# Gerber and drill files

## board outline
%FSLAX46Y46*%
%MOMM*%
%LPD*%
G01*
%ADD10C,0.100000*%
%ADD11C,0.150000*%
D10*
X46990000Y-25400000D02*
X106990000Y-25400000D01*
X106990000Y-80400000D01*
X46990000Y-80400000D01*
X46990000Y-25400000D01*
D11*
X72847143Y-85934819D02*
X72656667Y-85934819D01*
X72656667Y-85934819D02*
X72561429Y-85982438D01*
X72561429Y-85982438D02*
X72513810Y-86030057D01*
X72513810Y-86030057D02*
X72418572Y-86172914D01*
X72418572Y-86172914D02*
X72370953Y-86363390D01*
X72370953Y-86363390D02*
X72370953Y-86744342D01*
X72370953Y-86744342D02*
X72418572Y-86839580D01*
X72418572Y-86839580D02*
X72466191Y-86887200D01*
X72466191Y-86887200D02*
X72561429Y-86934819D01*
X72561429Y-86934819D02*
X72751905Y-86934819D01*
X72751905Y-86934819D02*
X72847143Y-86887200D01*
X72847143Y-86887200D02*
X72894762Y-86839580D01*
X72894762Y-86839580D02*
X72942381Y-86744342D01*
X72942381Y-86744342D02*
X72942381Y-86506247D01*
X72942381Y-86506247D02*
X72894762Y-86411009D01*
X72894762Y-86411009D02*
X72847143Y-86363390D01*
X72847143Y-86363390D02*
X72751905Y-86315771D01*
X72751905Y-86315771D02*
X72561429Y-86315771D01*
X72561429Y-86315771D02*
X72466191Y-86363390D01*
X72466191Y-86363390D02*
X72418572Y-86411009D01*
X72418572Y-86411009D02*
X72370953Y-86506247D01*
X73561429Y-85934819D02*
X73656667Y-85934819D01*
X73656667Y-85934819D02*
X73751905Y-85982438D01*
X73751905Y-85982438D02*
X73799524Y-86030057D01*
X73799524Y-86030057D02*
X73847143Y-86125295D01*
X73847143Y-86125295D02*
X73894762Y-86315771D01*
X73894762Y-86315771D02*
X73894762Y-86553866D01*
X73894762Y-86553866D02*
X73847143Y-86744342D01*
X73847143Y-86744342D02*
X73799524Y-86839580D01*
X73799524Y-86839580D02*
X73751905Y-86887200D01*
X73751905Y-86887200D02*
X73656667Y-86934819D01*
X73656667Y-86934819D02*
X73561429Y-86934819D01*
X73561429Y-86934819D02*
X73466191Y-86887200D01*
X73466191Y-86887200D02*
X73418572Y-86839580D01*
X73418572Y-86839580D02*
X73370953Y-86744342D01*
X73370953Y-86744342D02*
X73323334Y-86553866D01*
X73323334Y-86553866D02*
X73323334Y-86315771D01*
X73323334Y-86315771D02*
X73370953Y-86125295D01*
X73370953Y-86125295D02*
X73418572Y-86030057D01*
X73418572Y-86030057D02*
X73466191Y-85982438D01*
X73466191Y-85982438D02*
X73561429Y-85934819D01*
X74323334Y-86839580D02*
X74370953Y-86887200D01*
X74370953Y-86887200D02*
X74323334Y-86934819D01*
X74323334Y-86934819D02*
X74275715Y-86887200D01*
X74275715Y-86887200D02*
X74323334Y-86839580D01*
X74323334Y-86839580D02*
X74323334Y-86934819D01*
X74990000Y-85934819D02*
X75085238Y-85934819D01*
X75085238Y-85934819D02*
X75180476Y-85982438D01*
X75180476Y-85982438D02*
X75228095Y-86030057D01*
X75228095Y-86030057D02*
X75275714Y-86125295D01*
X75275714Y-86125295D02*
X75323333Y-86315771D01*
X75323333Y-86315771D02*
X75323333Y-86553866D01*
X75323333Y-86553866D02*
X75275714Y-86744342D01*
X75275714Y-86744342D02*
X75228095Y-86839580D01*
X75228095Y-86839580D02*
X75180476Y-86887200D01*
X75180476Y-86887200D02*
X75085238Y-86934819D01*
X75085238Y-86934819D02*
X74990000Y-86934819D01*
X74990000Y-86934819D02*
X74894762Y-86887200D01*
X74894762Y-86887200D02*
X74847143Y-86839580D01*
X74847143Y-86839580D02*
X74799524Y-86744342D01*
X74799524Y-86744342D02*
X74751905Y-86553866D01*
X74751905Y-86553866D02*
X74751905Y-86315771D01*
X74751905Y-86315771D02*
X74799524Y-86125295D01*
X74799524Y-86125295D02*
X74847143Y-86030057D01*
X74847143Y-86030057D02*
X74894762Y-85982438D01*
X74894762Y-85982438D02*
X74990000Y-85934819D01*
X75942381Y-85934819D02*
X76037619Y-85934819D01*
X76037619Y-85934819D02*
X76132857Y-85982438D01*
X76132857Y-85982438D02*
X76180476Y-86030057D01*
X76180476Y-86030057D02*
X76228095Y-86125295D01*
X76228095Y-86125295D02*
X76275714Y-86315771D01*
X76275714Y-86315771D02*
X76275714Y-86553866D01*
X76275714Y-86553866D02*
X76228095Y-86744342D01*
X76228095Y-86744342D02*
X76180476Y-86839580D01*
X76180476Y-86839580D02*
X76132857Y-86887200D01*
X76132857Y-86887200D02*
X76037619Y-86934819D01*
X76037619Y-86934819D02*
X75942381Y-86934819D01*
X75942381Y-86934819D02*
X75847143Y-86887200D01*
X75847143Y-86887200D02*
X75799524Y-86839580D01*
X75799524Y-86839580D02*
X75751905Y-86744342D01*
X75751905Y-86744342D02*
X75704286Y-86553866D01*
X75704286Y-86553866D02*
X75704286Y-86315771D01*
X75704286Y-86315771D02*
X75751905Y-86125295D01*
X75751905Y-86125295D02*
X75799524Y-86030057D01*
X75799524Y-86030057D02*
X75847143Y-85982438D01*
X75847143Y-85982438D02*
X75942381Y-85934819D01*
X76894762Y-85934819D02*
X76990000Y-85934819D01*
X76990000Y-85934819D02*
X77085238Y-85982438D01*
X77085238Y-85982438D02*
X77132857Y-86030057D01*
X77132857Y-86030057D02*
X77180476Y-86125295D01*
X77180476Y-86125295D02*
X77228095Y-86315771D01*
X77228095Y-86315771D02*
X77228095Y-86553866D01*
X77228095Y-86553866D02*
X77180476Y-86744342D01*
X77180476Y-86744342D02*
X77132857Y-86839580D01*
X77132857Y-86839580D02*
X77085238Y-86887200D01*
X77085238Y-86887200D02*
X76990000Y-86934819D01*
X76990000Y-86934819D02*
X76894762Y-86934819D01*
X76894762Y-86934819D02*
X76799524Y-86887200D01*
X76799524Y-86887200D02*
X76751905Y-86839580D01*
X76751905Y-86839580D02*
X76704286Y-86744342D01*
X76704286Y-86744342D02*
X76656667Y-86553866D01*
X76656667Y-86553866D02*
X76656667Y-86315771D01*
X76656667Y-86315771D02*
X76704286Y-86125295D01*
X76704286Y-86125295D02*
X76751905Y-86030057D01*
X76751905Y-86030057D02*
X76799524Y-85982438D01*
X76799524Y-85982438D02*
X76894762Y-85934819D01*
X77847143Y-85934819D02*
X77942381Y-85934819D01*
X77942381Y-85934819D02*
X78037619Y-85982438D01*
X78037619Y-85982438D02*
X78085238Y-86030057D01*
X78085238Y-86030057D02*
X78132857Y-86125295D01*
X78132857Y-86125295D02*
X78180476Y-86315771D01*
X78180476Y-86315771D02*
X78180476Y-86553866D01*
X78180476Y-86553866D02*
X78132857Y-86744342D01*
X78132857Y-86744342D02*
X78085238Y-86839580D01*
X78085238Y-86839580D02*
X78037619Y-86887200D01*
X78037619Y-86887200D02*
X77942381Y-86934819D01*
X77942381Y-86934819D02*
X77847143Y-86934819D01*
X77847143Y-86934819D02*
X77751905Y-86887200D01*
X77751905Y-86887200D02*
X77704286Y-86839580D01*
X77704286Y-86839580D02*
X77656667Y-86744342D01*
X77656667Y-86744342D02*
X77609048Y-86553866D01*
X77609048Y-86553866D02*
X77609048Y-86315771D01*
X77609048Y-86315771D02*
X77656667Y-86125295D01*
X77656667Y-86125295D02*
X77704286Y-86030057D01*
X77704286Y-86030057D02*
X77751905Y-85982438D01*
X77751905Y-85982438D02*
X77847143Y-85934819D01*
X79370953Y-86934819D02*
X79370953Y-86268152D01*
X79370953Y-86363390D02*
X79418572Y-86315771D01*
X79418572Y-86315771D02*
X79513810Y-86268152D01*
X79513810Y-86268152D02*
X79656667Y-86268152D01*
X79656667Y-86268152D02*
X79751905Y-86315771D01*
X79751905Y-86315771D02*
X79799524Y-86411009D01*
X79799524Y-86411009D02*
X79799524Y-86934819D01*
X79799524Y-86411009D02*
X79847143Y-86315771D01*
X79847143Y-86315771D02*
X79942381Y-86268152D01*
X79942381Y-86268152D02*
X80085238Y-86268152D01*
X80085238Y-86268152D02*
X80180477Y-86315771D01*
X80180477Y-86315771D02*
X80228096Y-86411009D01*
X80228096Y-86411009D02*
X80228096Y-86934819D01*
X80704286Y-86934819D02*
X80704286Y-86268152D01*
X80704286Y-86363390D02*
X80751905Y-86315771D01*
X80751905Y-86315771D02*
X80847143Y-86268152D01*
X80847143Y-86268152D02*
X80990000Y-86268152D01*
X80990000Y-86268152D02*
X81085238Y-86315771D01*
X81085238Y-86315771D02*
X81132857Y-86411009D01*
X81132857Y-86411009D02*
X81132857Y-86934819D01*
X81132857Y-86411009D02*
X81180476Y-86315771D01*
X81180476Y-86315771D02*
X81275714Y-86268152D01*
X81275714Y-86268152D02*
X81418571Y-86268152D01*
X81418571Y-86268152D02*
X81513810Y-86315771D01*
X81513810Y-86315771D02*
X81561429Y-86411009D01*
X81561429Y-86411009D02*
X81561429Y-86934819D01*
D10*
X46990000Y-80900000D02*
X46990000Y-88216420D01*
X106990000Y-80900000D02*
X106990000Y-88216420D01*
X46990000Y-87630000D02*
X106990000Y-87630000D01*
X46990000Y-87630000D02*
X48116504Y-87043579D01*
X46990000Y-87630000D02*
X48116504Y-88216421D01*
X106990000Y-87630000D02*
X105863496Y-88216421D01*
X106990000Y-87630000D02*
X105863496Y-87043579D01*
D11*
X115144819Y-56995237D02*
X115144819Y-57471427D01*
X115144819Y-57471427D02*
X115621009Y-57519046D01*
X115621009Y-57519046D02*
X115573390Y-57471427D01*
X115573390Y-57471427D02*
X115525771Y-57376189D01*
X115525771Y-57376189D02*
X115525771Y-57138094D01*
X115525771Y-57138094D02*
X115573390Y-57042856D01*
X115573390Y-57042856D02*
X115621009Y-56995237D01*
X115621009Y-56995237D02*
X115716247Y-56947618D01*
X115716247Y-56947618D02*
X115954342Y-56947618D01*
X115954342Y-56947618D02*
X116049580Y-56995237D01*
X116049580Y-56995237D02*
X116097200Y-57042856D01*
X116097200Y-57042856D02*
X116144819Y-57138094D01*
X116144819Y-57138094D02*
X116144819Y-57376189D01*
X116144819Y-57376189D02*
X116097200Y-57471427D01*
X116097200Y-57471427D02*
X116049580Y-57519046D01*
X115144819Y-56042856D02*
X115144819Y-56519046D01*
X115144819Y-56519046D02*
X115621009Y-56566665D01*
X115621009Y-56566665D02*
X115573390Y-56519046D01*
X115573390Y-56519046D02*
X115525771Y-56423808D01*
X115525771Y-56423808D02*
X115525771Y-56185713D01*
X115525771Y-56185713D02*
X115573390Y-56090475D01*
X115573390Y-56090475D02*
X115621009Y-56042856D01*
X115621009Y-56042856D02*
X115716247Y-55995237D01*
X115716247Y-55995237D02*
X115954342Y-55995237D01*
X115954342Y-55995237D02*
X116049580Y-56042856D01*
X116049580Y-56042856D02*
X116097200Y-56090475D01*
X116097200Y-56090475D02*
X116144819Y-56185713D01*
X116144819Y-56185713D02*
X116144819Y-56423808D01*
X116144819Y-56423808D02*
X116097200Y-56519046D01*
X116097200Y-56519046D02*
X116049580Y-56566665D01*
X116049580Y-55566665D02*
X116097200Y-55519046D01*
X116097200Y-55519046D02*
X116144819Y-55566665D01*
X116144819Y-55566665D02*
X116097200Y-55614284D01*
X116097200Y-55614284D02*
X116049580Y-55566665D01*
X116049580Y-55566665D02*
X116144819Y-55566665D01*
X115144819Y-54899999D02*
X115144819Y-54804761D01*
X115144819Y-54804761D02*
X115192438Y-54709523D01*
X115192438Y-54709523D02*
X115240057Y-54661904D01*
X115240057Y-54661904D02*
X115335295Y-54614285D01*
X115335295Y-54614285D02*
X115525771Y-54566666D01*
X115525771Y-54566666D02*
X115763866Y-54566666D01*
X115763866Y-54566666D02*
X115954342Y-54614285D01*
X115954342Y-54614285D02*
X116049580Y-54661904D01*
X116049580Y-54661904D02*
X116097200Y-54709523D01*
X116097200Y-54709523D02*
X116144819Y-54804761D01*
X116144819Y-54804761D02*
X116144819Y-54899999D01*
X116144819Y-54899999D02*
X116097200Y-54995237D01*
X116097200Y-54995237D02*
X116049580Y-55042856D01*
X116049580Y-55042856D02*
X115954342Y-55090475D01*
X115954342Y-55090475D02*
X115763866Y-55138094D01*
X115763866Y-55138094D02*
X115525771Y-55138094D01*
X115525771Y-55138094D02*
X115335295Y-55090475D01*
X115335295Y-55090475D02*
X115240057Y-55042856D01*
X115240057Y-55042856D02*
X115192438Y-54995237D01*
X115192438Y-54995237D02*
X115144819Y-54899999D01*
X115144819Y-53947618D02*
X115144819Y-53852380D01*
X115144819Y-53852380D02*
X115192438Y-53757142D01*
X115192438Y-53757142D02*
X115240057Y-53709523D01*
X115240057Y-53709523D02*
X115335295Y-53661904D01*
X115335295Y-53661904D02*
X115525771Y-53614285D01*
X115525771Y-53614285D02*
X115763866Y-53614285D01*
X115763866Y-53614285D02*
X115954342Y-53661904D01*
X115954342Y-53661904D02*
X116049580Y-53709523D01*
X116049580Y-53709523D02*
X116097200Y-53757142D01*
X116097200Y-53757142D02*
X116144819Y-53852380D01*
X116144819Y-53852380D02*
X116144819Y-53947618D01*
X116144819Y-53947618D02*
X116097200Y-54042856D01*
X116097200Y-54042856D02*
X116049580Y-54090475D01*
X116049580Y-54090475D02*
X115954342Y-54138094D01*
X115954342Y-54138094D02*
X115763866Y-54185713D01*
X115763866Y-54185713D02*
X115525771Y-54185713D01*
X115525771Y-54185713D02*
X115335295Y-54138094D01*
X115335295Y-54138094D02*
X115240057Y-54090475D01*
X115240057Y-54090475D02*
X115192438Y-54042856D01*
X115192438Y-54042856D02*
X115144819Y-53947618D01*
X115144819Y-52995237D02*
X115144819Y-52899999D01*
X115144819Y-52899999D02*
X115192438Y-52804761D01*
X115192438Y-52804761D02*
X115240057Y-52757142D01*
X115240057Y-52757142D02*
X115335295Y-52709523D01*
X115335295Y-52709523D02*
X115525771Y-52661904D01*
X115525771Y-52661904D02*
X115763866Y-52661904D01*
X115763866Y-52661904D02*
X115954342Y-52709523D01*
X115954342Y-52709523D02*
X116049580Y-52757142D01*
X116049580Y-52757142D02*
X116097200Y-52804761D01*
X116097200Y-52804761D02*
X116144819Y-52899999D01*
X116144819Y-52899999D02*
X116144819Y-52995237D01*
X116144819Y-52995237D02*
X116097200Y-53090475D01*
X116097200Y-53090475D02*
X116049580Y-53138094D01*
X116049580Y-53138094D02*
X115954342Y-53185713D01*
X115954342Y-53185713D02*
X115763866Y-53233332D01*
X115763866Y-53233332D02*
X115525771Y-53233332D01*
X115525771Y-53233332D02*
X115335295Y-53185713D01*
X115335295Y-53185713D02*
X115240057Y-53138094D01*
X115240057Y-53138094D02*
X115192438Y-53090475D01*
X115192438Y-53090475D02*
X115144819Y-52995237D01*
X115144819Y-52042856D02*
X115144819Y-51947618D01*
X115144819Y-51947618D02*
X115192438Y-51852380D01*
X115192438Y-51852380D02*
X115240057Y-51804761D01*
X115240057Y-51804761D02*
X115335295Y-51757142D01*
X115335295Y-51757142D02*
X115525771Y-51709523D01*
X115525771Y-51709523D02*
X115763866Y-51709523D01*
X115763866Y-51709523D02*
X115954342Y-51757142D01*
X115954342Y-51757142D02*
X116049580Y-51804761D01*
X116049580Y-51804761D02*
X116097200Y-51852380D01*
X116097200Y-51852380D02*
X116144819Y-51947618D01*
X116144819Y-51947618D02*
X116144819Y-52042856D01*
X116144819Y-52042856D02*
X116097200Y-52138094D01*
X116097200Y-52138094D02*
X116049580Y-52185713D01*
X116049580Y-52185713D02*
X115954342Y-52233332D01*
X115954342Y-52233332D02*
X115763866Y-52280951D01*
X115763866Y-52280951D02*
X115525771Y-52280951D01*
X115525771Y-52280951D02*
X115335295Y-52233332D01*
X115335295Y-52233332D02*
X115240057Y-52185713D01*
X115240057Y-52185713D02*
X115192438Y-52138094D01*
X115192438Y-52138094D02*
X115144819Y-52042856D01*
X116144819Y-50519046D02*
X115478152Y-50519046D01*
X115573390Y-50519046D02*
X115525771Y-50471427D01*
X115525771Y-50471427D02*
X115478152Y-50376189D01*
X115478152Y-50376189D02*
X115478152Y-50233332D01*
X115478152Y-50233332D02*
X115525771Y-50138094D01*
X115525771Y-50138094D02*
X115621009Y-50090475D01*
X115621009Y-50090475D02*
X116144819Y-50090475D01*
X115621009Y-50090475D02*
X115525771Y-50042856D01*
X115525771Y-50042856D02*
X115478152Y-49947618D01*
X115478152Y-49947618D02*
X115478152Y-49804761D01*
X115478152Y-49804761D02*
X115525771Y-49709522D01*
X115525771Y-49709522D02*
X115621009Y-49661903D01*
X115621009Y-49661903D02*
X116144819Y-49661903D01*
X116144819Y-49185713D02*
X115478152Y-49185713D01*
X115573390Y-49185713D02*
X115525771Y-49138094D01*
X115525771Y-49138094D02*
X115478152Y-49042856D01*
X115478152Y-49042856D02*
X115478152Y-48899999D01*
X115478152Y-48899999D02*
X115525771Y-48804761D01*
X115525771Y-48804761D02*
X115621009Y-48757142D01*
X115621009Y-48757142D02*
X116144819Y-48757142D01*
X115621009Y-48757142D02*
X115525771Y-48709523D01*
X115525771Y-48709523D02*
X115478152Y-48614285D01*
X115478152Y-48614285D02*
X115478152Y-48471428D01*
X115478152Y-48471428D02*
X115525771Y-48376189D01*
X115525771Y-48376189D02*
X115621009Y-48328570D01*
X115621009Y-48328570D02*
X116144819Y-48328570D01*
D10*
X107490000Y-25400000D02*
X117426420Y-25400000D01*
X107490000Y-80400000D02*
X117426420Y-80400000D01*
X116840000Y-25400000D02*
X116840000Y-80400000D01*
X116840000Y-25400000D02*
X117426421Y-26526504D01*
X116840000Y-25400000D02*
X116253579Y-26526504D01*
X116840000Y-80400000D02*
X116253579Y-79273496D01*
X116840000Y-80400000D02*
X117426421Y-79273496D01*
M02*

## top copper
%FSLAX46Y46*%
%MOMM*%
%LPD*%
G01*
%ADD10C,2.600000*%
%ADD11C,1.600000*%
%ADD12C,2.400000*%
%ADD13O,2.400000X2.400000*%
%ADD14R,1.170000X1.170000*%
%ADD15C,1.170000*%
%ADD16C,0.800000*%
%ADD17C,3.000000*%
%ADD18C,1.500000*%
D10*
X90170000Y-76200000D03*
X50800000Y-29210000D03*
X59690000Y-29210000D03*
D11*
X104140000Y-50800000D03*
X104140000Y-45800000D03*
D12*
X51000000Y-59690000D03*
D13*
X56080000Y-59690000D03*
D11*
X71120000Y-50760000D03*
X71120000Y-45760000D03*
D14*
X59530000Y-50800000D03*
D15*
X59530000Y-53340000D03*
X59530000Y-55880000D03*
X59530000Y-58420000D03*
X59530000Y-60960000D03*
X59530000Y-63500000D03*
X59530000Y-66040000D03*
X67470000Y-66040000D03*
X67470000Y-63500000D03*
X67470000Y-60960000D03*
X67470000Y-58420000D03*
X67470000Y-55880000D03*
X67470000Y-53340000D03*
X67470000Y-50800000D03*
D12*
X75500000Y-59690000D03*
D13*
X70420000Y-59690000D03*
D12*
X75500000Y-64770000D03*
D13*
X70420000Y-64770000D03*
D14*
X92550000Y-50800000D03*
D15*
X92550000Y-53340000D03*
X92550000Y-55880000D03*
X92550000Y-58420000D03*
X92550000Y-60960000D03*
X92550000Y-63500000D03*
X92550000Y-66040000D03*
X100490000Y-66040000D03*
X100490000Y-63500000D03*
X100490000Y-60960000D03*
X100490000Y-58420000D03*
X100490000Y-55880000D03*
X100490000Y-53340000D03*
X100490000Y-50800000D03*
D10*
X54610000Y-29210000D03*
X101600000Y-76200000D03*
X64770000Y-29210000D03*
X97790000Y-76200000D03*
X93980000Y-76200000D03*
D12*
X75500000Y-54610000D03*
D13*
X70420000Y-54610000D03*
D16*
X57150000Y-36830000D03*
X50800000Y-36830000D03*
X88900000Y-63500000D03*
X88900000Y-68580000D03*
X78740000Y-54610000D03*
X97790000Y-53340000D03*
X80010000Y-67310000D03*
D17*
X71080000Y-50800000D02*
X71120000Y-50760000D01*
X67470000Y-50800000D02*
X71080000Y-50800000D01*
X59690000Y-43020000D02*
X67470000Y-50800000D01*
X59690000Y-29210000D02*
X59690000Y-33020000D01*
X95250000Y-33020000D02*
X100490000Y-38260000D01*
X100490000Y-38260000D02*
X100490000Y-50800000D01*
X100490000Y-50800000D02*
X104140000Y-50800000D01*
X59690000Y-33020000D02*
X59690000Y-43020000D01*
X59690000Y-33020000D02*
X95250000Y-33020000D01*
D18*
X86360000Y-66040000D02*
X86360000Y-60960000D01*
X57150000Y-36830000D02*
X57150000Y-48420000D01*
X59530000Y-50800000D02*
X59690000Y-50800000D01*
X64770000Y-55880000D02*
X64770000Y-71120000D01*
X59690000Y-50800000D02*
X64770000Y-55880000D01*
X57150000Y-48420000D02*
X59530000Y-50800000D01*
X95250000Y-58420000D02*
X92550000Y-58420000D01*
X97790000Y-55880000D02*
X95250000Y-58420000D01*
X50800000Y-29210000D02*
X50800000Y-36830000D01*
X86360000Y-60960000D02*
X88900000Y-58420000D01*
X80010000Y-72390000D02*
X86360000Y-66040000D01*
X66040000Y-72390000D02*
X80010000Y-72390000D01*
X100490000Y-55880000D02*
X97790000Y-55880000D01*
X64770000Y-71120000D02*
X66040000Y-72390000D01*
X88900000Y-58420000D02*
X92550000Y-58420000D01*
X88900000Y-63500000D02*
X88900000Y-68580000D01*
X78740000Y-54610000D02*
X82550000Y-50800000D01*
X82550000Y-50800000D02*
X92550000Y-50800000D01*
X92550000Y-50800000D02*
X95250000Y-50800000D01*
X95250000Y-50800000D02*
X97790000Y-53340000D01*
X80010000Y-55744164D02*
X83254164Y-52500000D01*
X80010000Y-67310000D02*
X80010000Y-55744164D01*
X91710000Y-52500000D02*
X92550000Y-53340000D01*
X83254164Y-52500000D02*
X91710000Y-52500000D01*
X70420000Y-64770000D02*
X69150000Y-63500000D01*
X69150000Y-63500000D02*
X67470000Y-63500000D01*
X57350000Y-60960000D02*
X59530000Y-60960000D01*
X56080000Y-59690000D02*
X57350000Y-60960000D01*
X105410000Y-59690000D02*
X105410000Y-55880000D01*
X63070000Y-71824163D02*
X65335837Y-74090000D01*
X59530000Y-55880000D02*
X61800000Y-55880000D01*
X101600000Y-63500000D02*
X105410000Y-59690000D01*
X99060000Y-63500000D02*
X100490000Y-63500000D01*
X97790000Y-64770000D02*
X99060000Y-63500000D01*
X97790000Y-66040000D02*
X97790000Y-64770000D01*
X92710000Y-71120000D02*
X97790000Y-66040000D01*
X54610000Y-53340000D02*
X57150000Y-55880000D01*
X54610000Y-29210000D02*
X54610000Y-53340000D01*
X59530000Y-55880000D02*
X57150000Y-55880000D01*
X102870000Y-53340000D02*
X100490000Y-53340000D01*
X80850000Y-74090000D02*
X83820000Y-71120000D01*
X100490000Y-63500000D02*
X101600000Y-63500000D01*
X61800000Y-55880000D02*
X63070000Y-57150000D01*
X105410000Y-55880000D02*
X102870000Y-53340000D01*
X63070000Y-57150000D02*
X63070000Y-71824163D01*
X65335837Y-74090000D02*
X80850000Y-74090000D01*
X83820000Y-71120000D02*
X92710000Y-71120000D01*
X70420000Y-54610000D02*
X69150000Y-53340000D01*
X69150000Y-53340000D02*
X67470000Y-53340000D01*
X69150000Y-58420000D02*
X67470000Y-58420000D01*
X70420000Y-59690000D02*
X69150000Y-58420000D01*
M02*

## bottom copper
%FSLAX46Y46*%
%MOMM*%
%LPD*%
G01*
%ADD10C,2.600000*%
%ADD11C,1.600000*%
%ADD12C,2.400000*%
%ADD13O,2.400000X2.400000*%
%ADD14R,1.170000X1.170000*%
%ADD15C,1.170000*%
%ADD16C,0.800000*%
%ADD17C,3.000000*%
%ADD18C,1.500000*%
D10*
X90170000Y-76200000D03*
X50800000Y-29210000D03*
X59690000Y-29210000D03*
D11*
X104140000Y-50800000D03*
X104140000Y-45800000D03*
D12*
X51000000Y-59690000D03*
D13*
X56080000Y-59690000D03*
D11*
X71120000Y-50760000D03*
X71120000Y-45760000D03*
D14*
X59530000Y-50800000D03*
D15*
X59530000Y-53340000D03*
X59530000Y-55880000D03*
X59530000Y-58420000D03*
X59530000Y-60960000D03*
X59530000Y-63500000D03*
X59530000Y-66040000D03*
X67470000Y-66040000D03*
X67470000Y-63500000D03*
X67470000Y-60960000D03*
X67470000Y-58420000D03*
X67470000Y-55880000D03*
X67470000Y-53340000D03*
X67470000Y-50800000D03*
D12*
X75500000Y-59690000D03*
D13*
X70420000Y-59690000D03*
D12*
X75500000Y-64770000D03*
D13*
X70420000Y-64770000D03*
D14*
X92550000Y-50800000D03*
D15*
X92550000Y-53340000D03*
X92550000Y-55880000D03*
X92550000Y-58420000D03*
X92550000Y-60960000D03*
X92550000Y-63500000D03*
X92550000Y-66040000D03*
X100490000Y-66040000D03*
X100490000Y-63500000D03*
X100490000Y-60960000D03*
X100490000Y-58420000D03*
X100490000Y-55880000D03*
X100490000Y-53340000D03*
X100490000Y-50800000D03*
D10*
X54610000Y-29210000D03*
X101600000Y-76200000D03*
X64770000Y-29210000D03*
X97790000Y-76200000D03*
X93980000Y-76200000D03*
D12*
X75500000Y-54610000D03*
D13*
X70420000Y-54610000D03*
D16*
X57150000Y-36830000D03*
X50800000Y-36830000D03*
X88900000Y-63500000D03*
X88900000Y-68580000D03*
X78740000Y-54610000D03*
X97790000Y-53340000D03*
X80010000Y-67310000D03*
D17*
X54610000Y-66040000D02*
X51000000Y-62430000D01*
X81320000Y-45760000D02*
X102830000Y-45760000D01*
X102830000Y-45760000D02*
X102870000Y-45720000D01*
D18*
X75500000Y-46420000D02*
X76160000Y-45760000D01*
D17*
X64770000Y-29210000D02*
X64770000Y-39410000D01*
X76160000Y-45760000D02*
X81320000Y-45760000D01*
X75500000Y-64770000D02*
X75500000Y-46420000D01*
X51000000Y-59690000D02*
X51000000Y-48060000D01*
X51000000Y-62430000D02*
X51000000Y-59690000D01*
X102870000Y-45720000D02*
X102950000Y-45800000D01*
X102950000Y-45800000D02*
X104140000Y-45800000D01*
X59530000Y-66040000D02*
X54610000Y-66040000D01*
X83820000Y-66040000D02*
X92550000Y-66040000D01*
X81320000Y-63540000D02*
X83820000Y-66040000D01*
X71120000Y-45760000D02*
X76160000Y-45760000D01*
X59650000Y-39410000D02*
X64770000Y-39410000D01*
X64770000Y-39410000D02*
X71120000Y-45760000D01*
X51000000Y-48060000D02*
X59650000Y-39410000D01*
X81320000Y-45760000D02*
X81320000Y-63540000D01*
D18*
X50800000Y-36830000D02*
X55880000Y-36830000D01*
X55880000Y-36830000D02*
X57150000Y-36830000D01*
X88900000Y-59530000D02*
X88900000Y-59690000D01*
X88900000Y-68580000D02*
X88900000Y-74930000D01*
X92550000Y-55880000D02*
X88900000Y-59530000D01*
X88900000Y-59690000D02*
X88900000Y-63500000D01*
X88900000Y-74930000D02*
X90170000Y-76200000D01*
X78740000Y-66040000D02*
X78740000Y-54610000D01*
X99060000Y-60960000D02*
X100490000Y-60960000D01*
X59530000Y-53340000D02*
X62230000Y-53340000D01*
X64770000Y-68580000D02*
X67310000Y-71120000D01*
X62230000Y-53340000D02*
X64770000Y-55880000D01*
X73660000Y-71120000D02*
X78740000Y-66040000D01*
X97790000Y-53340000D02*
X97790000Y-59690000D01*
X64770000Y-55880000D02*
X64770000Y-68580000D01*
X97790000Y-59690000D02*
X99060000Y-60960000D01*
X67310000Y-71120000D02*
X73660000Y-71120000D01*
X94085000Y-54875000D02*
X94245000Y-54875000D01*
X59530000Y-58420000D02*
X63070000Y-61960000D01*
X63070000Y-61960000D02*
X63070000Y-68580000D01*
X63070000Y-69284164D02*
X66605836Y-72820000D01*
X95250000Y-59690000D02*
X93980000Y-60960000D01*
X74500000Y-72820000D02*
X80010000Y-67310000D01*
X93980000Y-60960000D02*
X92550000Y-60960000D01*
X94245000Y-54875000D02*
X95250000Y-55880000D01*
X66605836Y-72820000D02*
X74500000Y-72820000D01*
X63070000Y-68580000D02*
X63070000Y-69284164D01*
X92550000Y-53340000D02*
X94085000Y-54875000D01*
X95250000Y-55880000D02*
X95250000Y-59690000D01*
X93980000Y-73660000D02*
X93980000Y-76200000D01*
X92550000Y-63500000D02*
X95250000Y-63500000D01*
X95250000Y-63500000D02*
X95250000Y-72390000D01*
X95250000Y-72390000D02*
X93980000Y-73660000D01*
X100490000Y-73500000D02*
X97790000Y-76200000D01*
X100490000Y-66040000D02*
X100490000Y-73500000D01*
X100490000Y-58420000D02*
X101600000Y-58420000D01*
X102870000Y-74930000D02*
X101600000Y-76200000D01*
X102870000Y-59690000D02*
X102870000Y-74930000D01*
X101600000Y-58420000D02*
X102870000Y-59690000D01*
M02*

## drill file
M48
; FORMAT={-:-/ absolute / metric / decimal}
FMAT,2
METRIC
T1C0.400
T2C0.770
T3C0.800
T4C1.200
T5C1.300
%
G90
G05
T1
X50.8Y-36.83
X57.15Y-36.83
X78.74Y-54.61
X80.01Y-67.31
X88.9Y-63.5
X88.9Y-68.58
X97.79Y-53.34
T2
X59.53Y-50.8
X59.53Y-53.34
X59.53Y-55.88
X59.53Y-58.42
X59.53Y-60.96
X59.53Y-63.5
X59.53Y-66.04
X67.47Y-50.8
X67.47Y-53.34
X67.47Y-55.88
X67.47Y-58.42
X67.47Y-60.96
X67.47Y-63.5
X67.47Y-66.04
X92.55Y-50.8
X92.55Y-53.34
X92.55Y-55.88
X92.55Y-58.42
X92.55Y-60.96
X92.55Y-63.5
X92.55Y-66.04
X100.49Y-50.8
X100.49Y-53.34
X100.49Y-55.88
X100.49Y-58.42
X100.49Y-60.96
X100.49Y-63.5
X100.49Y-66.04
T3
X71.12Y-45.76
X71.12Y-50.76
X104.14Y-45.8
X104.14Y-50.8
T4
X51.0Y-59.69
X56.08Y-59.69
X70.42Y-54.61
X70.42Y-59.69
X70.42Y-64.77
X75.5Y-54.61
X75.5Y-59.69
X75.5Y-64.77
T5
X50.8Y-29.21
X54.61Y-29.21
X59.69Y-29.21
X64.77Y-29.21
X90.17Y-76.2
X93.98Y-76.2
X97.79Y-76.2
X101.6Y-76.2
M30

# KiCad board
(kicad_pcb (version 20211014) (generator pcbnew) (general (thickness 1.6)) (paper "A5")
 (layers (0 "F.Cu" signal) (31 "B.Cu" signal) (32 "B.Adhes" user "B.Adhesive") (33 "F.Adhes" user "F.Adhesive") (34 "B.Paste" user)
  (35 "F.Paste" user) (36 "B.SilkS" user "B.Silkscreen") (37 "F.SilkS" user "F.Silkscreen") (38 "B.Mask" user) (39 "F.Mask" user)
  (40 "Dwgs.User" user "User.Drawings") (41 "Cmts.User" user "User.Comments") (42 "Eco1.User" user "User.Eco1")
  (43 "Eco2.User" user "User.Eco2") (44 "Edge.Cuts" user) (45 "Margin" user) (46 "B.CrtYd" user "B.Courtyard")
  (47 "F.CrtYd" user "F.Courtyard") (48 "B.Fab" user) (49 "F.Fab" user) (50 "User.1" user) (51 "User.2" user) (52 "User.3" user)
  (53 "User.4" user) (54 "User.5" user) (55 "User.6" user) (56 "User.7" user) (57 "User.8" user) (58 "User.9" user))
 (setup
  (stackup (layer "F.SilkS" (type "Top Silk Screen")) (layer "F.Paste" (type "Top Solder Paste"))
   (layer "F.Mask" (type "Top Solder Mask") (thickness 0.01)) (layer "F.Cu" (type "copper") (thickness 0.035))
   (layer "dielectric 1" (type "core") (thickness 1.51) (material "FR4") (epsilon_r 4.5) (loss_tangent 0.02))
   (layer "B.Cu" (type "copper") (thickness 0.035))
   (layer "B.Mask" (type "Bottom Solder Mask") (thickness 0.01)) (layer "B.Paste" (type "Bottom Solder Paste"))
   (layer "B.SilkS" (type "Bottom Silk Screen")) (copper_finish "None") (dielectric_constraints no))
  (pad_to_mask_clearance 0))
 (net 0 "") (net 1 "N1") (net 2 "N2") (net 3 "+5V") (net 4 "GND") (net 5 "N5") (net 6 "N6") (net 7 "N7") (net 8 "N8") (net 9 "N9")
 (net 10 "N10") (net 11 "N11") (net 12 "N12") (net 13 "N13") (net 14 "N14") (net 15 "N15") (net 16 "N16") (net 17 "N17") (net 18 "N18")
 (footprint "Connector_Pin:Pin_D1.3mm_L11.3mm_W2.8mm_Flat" (layer "F.Cu") (at 90.17 76.2)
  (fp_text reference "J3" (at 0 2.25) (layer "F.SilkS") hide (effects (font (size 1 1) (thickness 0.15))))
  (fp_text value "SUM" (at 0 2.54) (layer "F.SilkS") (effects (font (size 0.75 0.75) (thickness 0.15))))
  (pad "1" thru_hole circle (at 0 0) (size 2.6 2.6) (drill 1.3) (layers *.Cu *.Mask) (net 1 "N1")))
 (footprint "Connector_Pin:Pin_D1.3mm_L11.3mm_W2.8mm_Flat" (layer "F.Cu") (at 50.8 29.21)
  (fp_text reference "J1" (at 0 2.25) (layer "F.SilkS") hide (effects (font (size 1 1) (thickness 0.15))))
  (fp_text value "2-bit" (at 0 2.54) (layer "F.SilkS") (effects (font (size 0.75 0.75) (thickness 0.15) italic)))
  (pad "1" thru_hole circle (at 0 0) (size 2.6 2.6) (drill 1.3) (layers *.Cu *.Mask) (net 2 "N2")))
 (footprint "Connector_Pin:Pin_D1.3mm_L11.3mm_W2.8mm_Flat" (layer "F.Cu") (at 59.69 29.21)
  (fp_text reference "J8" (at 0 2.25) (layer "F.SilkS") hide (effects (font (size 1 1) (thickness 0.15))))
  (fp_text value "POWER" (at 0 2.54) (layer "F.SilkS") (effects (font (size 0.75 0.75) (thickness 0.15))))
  (pad "1" thru_hole circle (at 0 0) (size 2.6 2.6) (drill 1.3) (layers *.Cu *.Mask) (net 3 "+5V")))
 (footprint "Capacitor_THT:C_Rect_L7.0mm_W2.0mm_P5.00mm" (layer "F.Cu") (at 104.14 50.8 90)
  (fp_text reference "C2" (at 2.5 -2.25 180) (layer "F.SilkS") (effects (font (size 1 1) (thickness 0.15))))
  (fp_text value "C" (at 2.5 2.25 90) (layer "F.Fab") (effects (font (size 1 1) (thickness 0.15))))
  (pad "1" thru_hole circle (at 0 0 90) (size 1.6 1.6) (drill 0.8) (layers *.Cu *.Mask) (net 3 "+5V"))
  (pad "2" thru_hole circle (at 5 0 90) (size 1.6 1.6) (drill 0.8) (layers *.Cu *.Mask) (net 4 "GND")))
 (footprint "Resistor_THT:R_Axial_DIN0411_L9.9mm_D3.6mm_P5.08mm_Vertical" (layer "F.Cu") (at 51 59.69)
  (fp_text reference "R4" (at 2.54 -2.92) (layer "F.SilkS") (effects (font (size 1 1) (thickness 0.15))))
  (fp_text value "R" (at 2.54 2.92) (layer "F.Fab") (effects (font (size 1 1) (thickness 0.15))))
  (pad "1" thru_hole circle (at 0 0) (size 2.4 2.4) (drill 1.2) (layers *.Cu *.Mask) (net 4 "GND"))
  (pad "2" thru_hole oval (at 5.08 0) (size 2.4 2.4) (drill 1.2) (layers *.Cu *.Mask) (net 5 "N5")))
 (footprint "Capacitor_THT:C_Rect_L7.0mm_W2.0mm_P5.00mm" (layer "F.Cu") (at 71.12 50.76 90)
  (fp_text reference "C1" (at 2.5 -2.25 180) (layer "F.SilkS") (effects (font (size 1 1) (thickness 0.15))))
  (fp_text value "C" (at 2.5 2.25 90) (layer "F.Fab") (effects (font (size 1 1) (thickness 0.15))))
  (pad "1" thru_hole circle (at 0 0 90) (size 1.6 1.6) (drill 0.8) (layers *.Cu *.Mask) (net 3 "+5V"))
  (pad "2" thru_hole circle (at 5 0 90) (size 1.6 1.6) (drill 0.8) (layers *.Cu *.Mask) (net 4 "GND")))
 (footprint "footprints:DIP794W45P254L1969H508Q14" (layer "F.Cu") (at 63.5 58.42)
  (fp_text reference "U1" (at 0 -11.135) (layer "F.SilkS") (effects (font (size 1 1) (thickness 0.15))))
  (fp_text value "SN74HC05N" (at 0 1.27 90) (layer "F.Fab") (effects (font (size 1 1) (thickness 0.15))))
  (pad "1" thru_hole rect locked (at -3.97 -7.62) (size 1.17 1.17) (drill 0.77) (layers *.Cu *.Mask) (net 2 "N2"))
  (pad "2" thru_hole circle locked (at -3.97 -5.08) (size 1.17 1.17) (drill 0.77) (layers *.Cu *.Mask) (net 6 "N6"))
  (pad "3" thru_hole circle locked (at -3.97 -2.54) (size 1.17 1.17) (drill 0.77) (layers *.Cu *.Mask) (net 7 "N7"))
  (pad "4" thru_hole circle locked (at -3.97 0) (size 1.17 1.17) (drill 0.77) (layers *.Cu *.Mask) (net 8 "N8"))
  (pad "5" thru_hole circle locked (at -3.97 2.54) (size 1.17 1.17) (drill 0.77) (layers *.Cu *.Mask) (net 5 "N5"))
  (pad "6" thru_hole circle locked (at -3.97 5.08) (size 1.17 1.17) (drill 0.77) (layers *.Cu *.Mask) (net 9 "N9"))
  (pad "7" thru_hole circle locked (at -3.97 7.62) (size 1.17 1.17) (drill 0.77) (layers *.Cu *.Mask) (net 4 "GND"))
  (pad "8" thru_hole circle locked (at 3.97 7.62) (size 1.17 1.17) (drill 0.77) (layers *.Cu *.Mask) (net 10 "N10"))
  (pad "9" thru_hole circle locked (at 3.97 5.08) (size 1.17 1.17) (drill 0.77) (layers *.Cu *.Mask) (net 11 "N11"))
  (pad "10" thru_hole circle locked (at 3.97 2.54) (size 1.17 1.17) (drill 0.77) (layers *.Cu *.Mask) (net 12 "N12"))
  (pad "11" thru_hole circle locked (at 3.97 0) (size 1.17 1.17) (drill 0.77) (layers *.Cu *.Mask) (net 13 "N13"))
  (pad "12" thru_hole circle locked (at 3.97 -2.54) (size 1.17 1.17) (drill 0.77) (layers *.Cu *.Mask) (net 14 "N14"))
  (pad "13" thru_hole circle locked (at 3.97 -5.08) (size 1.17 1.17) (drill 0.77) (layers *.Cu *.Mask) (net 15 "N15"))
  (pad "14" thru_hole circle locked (at 3.97 -7.62) (size 1.17 1.17) (drill 0.77) (layers *.Cu *.Mask) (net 3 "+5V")))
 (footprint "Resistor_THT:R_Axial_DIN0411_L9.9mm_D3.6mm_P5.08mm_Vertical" (layer "F.Cu") (at 75.5 59.69 180)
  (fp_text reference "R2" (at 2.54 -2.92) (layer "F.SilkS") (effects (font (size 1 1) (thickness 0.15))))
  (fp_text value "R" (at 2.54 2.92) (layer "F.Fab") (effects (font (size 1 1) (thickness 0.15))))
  (pad "1" thru_hole circle (at 0 0 180) (size 2.4 2.4) (drill 1.2) (layers *.Cu *.Mask) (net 4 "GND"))
  (pad "2" thru_hole oval (at 5.08 0 180) (size 2.4 2.4) (drill 1.2) (layers *.Cu *.Mask) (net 13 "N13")))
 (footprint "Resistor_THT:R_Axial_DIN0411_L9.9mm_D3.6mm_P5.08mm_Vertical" (layer "F.Cu") (at 75.5 64.77 180)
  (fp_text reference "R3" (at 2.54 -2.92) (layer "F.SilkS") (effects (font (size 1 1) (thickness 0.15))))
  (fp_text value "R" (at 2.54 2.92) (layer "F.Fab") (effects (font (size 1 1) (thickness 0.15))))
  (pad "1" thru_hole circle (at 0 0 180) (size 2.4 2.4) (drill 1.2) (layers *.Cu *.Mask) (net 4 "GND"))
  (pad "2" thru_hole oval (at 5.08 0 180) (size 2.4 2.4) (drill 1.2) (layers *.Cu *.Mask) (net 11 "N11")))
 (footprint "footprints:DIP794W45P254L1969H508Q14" (layer "F.Cu") (at 96.52 58.42)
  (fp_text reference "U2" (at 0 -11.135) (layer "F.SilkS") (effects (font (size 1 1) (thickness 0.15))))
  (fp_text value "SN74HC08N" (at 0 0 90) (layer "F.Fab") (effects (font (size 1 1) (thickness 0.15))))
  (pad "1" thru_hole rect locked (at -3.97 -7.62) (size 1.17 1.17) (drill 0.77) (layers *.Cu *.Mask) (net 6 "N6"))
  (pad "2" thru_hole circle locked (at -3.97 -5.08) (size 1.17 1.17) (drill 0.77) (layers *.Cu *.Mask) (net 8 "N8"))
  (pad "3" thru_hole circle locked (at -3.97 -2.54) (size 1.17 1.17) (drill 0.77) (layers *.Cu *.Mask) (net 1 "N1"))
  (pad "4" thru_hole circle locked (at -3.97 0) (size 1.17 1.17) (drill 0.77) (layers *.Cu *.Mask) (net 2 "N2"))
  (pad "5" thru_hole circle locked (at -3.97 2.54) (size 1.17 1.17) (drill 0.77) (layers *.Cu *.Mask) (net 8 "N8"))
  (pad "6" thru_hole circle locked (at -3.97 5.08) (size 1.17 1.17) (drill 0.77) (layers *.Cu *.Mask) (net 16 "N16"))
  (pad "7" thru_hole circle locked (at -3.97 7.62) (size 1.17 1.17) (drill 0.77) (layers *.Cu *.Mask) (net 4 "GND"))
  (pad "8" thru_hole circle locked (at 3.97 7.62) (size 1.17 1.17) (drill 0.77) (layers *.Cu *.Mask) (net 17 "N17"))
  (pad "9" thru_hole circle locked (at 3.97 5.08) (size 1.17 1.17) (drill 0.77) (layers *.Cu *.Mask) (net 7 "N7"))
  (pad "10" thru_hole circle locked (at 3.97 2.54) (size 1.17 1.17) (drill 0.77) (layers *.Cu *.Mask) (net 6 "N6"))
  (pad "11" thru_hole circle locked (at 3.97 0) (size 1.17 1.17) (drill 0.77) (layers *.Cu *.Mask) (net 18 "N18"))
  (pad "12" thru_hole circle locked (at 3.97 -2.54) (size 1.17 1.17) (drill 0.77) (layers *.Cu *.Mask) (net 2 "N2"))
  (pad "13" thru_hole circle locked (at 3.97 -5.08) (size 1.17 1.17) (drill 0.77) (layers *.Cu *.Mask) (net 7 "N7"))
  (pad "14" thru_hole circle locked (at 3.97 -7.62) (size 1.17 1.17) (drill 0.77) (layers *.Cu *.Mask) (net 3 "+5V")))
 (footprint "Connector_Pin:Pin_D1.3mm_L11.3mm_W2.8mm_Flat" (layer "F.Cu") (at 54.61 29.21)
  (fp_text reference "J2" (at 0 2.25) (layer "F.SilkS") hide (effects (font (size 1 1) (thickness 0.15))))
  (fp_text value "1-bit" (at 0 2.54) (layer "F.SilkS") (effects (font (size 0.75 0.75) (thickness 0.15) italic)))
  (pad "1" thru_hole circle (at 0 0) (size 2.6 2.6) (drill 1.3) (layers *.Cu *.Mask) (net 7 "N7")))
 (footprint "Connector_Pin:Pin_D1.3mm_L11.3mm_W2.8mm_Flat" (layer "F.Cu") (at 101.6 76.2)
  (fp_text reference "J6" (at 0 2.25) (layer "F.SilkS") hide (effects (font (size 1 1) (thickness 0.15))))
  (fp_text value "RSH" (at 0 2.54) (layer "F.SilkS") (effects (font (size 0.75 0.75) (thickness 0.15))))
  (pad "1" thru_hole circle (at 0 0) (size 2.6 2.6) (drill 1.3) (layers *.Cu *.Mask) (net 18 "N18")))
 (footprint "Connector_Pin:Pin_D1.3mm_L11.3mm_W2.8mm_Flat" (layer "F.Cu") (at 64.77 29.21)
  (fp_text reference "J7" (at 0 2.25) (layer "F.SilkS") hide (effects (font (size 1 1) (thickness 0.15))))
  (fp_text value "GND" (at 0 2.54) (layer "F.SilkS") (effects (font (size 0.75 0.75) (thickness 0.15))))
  (pad "1" thru_hole circle (at 0 0) (size 2.6 2.6) (drill 1.3) (layers *.Cu *.Mask) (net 4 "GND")))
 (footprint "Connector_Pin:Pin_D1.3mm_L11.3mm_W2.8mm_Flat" (layer "F.Cu") (at 97.79 76.2)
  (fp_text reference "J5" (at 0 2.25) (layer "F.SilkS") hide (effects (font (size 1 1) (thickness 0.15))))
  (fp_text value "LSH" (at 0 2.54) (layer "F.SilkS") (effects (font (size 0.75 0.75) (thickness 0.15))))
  (pad "1" thru_hole circle (at 0 0) (size 2.6 2.6) (drill 1.3) (layers *.Cu *.Mask) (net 17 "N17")))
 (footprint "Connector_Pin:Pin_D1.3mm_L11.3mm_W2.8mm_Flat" (layer "F.Cu") (at 93.98 76.2)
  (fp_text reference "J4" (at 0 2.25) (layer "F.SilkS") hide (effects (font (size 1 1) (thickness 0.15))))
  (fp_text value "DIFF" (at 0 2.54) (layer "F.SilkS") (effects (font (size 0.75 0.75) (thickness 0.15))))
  (pad "1" thru_hole circle (at 0 0) (size 2.6 2.6) (drill 1.3) (layers *.Cu *.Mask) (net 16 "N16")))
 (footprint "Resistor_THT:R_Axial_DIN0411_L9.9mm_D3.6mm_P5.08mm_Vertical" (layer "F.Cu") (at 75.5 54.61 180)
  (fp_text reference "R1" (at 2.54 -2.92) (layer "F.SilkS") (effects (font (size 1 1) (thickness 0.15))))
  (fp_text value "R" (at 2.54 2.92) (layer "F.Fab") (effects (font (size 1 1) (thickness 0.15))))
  (pad "1" thru_hole circle (at 0 0 180) (size 2.4 2.4) (drill 1.2) (layers *.Cu *.Mask) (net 4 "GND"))
  (pad "2" thru_hole oval (at 5.08 0 180) (size 2.4 2.4) (drill 1.2) (layers *.Cu *.Mask) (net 15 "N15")))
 (gr_rect (start 46.99 25.4) (end 106.99 80.4) (layer "Edge.Cuts") (width 0.1) (fill none))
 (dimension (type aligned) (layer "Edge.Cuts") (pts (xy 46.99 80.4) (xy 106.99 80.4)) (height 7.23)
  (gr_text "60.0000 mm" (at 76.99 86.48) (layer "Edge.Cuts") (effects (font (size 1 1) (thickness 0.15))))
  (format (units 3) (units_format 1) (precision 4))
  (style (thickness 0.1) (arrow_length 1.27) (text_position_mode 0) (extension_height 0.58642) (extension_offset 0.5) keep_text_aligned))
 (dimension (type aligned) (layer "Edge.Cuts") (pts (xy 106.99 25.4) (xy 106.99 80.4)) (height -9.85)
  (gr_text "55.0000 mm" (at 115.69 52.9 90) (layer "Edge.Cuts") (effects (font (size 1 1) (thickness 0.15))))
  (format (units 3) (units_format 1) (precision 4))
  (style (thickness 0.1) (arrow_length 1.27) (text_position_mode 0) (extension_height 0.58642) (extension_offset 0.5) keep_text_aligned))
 (segment (start 71.08 50.8) (end 71.12 50.76) (width 3) (layer "F.Cu") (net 3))
 (segment (start 67.47 50.8) (end 71.08 50.8) (width 3) (layer "F.Cu") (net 3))
 (segment (start 59.69 43.02) (end 67.47 50.8) (width 3) (layer "F.Cu") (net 3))
 (segment (start 59.69 29.21) (end 59.69 33.02) (width 3) (layer "F.Cu") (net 3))
 (segment (start 95.25 33.02) (end 100.49 38.26) (width 3) (layer "F.Cu") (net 3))
 (segment (start 100.49 38.26) (end 100.49 50.8) (width 3) (layer "F.Cu") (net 3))
 (segment (start 100.49 50.8) (end 104.14 50.8) (width 3) (layer "F.Cu") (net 3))
 (segment (start 59.69 33.02) (end 59.69 43.02) (width 3) (layer "F.Cu") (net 3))
 (segment (start 59.69 33.02) (end 95.25 33.02) (width 3) (layer "F.Cu") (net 3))
 (segment (start 54.61 66.04) (end 51 62.43) (width 3) (layer "B.Cu") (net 4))
 (segment (start 81.32 45.76) (end 102.83 45.76) (width 3) (layer "B.Cu") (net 4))
 (segment (start 102.83 45.76) (end 102.87 45.72) (width 3) (layer "B.Cu") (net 4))
 (segment (start 75.5 46.42) (end 76.16 45.76) (width 1.5) (layer "B.Cu") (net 4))
 (segment (start 64.77 29.21) (end 64.77 39.41) (width 3) (layer "B.Cu") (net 4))
 (segment (start 76.16 45.76) (end 81.32 45.76) (width 3) (layer "B.Cu") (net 4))
 (segment (start 75.5 64.77) (end 75.5 46.42) (width 3) (layer "B.Cu") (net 4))
 (segment (start 51 59.69) (end 51 48.06) (width 3) (layer "B.Cu") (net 4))
 (segment (start 51 62.43) (end 51 59.69) (width 3) (layer "B.Cu") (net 4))
 (segment (start 102.87 45.72) (end 102.95 45.8) (width 3) (layer "B.Cu") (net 4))
 (segment (start 102.95 45.8) (end 104.14 45.8) (width 3) (layer "B.Cu") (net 4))
 (segment (start 59.53 66.04) (end 54.61 66.04) (width 3) (layer "B.Cu") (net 4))
 (segment (start 83.82 66.04) (end 92.55 66.04) (width 3) (layer "B.Cu") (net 4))
 (segment (start 81.32 63.54) (end 83.82 66.04) (width 3) (layer "B.Cu") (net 4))
 (segment (start 71.12 45.76) (end 76.16 45.76) (width 3) (layer "B.Cu") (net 4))
 (segment (start 59.65 39.41) (end 64.77 39.41) (width 3) (layer "B.Cu") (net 4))
 (segment (start 64.77 39.41) (end 71.12 45.76) (width 3) (layer "B.Cu") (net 4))
 (segment (start 51 48.06) (end 59.65 39.41) (width 3) (layer "B.Cu") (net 4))
 (segment (start 81.32 45.76) (end 81.32 63.54) (width 3) (layer "B.Cu") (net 4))
 (segment (start 86.36 66.04) (end 86.36 60.96) (width 1.5) (layer "F.Cu") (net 2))
 (segment (start 57.15 36.83) (end 57.15 48.42) (width 1.5) (layer "F.Cu") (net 2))
 (segment (start 59.53 50.8) (end 59.69 50.8) (width 1.5) (layer "F.Cu") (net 2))
 (segment (start 64.77 55.88) (end 64.77 71.12) (width 1.5) (layer "F.Cu") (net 2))
 (segment (start 59.69 50.8) (end 64.77 55.88) (width 1.5) (layer "F.Cu") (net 2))
 (segment (start 57.15 48.42) (end 59.53 50.8) (width 1.5) (layer "F.Cu") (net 2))
 (segment (start 95.25 58.42) (end 92.55 58.42) (width 1.5) (layer "F.Cu") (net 2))
 (segment (start 97.79 55.88) (end 95.25 58.42) (width 1.5) (layer "F.Cu") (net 2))
 (segment (start 50.8 29.21) (end 50.8 36.83) (width 1.5) (layer "F.Cu") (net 2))
 (segment (start 86.36 60.96) (end 88.9 58.42) (width 1.5) (layer "F.Cu") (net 2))
 (segment (start 80.01 72.39) (end 86.36 66.04) (width 1.5) (layer "F.Cu") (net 2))
 (segment (start 66.04 72.39) (end 80.01 72.39) (width 1.5) (layer "F.Cu") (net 2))
 (segment (start 100.49 55.88) (end 97.79 55.88) (width 1.5) (layer "F.Cu") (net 2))
 (segment (start 64.77 71.12) (end 66.04 72.39) (width 1.5) (layer "F.Cu") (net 2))
 (segment (start 88.9 58.42) (end 92.55 58.42) (width 1.5) (layer "F.Cu") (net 2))
 (via (at 57.15 36.83) (size 0.8) (drill 0.4) (layers "F.Cu" "B.Cu") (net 2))
 (via (at 50.8 36.83) (size 0.8) (drill 0.4) (layers "F.Cu" "B.Cu") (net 2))
 (segment (start 50.8 36.83) (end 55.88 36.83) (width 1.5) (layer "B.Cu") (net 2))
 (segment (start 55.88 36.83) (end 57.15 36.83) (width 1.5) (layer "B.Cu") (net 2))
 (segment (start 88.9 63.5) (end 88.9 68.58) (width 1.5) (layer "F.Cu") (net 1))
 (via (at 88.9 63.5) (size 0.8) (drill 0.4) (layers "F.Cu" "B.Cu") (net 1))
 (via (at 88.9 68.58) (size 0.8) (drill 0.4) (layers "F.Cu" "B.Cu") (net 1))
 (segment (start 88.9 59.53) (end 88.9 59.69) (width 1.5) (layer "B.Cu") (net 1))
 (segment (start 88.9 68.58) (end 88.9 74.93) (width 1.5) (layer "B.Cu") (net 1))
 (segment (start 92.55 55.88) (end 88.9 59.53) (width 1.5) (layer "B.Cu") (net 1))
 (segment (start 88.9 59.69) (end 88.9 63.5) (width 1.5) (layer "B.Cu") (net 1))
 (segment (start 88.9 74.93) (end 90.17 76.2) (width 1.5) (layer "B.Cu") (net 1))
 (segment (start 78.74 54.61) (end 82.55 50.8) (width 1.5) (layer "F.Cu") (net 6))
 (segment (start 82.55 50.8) (end 92.55 50.8) (width 1.5) (layer "F.Cu") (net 6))
 (segment (start 92.55 50.8) (end 95.25 50.8) (width 1.5) (layer "F.Cu") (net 6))
 (segment (start 95.25 50.8) (end 97.79 53.34) (width 1.5) (layer "F.Cu") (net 6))
 (via (at 78.74 54.61) (size 0.8) (drill 0.4) (layers "F.Cu" "B.Cu") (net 6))
 (via (at 97.79 53.34) (size 0.8) (drill 0.4) (layers "F.Cu" "B.Cu") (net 6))
 (segment (start 78.74 66.04) (end 78.74 54.61) (width 1.5) (layer "B.Cu") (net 6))
 (segment (start 99.06 60.96) (end 100.49 60.96) (width 1.5) (layer "B.Cu") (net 6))
 (segment (start 59.53 53.34) (end 62.23 53.34) (width 1.5) (layer "B.Cu") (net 6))
 (segment (start 64.77 68.58) (end 67.31 71.12) (width 1.5) (layer "B.Cu") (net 6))
 (segment (start 62.23 53.34) (end 64.77 55.88) (width 1.5) (layer "B.Cu") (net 6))
 (segment (start 73.66 71.12) (end 78.74 66.04) (width 1.5) (layer "B.Cu") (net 6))
 (segment (start 97.79 53.34) (end 97.79 59.69) (width 1.5) (layer "B.Cu") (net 6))
 (segment (start 64.77 55.88) (end 64.77 68.58) (width 1.5) (layer "B.Cu") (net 6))
 (segment (start 97.79 59.69) (end 99.06 60.96) (width 1.5) (layer "B.Cu") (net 6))
 (segment (start 67.31 71.12) (end 73.66 71.12) (width 1.5) (layer "B.Cu") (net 6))
 (segment (start 80.01 55.744164) (end 83.254164 52.5) (width 1.5) (layer "F.Cu") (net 8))
 (segment (start 80.01 67.31) (end 80.01 55.744164) (width 1.5) (layer "F.Cu") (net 8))
 (segment (start 91.71 52.5) (end 92.55 53.34) (width 1.5) (layer "F.Cu") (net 8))
 (segment (start 83.254164 52.5) (end 91.71 52.5) (width 1.5) (layer "F.Cu") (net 8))
 (via (at 80.01 67.31) (size 0.8) (drill 0.4) (layers "F.Cu" "B.Cu") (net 8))
 (segment (start 94.085 54.875) (end 94.245 54.875) (width 1.5) (layer "B.Cu") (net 8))
 (segment (start 59.53 58.42) (end 63.07 61.96) (width 1.5) (layer "B.Cu") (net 8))
 (segment (start 63.07 61.96) (end 63.07 68.58) (width 1.5) (layer "B.Cu") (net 8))
 (segment (start 63.07 69.284164) (end 66.605836 72.82) (width 1.5) (layer "B.Cu") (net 8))
 (segment (start 95.25 59.69) (end 93.98 60.96) (width 1.5) (layer "B.Cu") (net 8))
 (segment (start 74.5 72.82) (end 80.01 67.31) (width 1.5) (layer "B.Cu") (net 8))
 (segment (start 93.98 60.96) (end 92.55 60.96) (width 1.5) (layer "B.Cu") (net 8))
 (segment (start 94.245 54.875) (end 95.25 55.88) (width 1.5) (layer "B.Cu") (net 8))
 (segment (start 66.605836 72.82) (end 74.5 72.82) (width 1.5) (layer "B.Cu") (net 8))
 (segment (start 63.07 68.58) (end 63.07 69.284164) (width 1.5) (layer "B.Cu") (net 8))
 (segment (start 92.55 53.34) (end 94.085 54.875) (width 1.5) (layer "B.Cu") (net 8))
 (segment (start 95.25 55.88) (end 95.25 59.69) (width 1.5) (layer "B.Cu") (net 8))
 (segment (start 70.42 64.77) (end 69.15 63.5) (width 1.5) (layer "F.Cu") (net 11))
 (segment (start 69.15 63.5) (end 67.47 63.5) (width 1.5) (layer "F.Cu") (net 11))
 (segment (start 57.35 60.96) (end 59.53 60.96) (width 1.5) (layer "F.Cu") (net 5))
 (segment (start 56.08 59.69) (end 57.35 60.96) (width 1.5) (layer "F.Cu") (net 5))
 (segment (start 93.98 73.66) (end 93.98 76.2) (width 1.5) (layer "B.Cu") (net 16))
 (segment (start 92.55 63.5) (end 95.25 63.5) (width 1.5) (layer "B.Cu") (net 16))
 (segment (start 95.25 63.5) (end 95.25 72.39) (width 1.5) (layer "B.Cu") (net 16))
 (segment (start 95.25 72.39) (end 93.98 73.66) (width 1.5) (layer "B.Cu") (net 16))
 (segment (start 105.41 59.69) (end 105.41 55.88) (width 1.5) (layer "F.Cu") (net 7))
 (segment (start 63.07 71.824163) (end 65.335837 74.09) (width 1.5) (layer "F.Cu") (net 7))
 (segment (start 59.53 55.88) (end 61.8 55.88) (width 1.5) (layer "F.Cu") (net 7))
 (segment (start 101.6 63.5) (end 105.41 59.69) (width 1.5) (layer "F.Cu") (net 7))
 (segment (start 99.06 63.5) (end 100.49 63.5) (width 1.5) (layer "F.Cu") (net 7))
 (segment (start 97.79 64.77) (end 99.06 63.5) (width 1.5) (layer "F.Cu") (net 7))
 (segment (start 97.79 66.04) (end 97.79 64.77) (width 1.5) (layer "F.Cu") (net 7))
 (segment (start 92.71 71.12) (end 97.79 66.04) (width 1.5) (layer "F.Cu") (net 7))
 (segment (start 54.61 53.34) (end 57.15 55.88) (width 1.5) (layer "F.Cu") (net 7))
 (segment (start 54.61 29.21) (end 54.61 53.34) (width 1.5) (layer "F.Cu") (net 7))
 (segment (start 59.53 55.88) (end 57.15 55.88) (width 1.5) (layer "F.Cu") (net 7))
 (segment (start 102.87 53.34) (end 100.49 53.34) (width 1.5) (layer "F.Cu") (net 7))
 (segment (start 80.85 74.09) (end 83.82 71.12) (width 1.5) (layer "F.Cu") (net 7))
 (segment (start 100.49 63.5) (end 101.6 63.5) (width 1.5) (layer "F.Cu") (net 7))
 (segment (start 61.8 55.88) (end 63.07 57.15) (width 1.5) (layer "F.Cu") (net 7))
 (segment (start 105.41 55.88) (end 102.87 53.34) (width 1.5) (layer "F.Cu") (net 7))
 (segment (start 63.07 57.15) (end 63.07 71.824163) (width 1.5) (layer "F.Cu") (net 7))
 (segment (start 65.335837 74.09) (end 80.85 74.09) (width 1.5) (layer "F.Cu") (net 7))
 (segment (start 83.82 71.12) (end 92.71 71.12) (width 1.5) (layer "F.Cu") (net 7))
 (segment (start 100.49 73.5) (end 97.79 76.2) (width 1.5) (layer "B.Cu") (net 17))
 (segment (start 100.49 66.04) (end 100.49 73.5) (width 1.5) (layer "B.Cu") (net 17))
 (segment (start 100.49 58.42) (end 101.6 58.42) (width 1.5) (layer "B.Cu") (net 18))
 (segment (start 102.87 74.93) (end 101.6 76.2) (width 1.5) (layer "B.Cu") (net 18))
 (segment (start 102.87 59.69) (end 102.87 74.93) (width 1.5) (layer "B.Cu") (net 18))
 (segment (start 101.6 58.42) (end 102.87 59.69) (width 1.5) (layer "B.Cu") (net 18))
 (segment (start 70.42 54.61) (end 69.15 53.34) (width 1.5) (layer "F.Cu") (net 15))
 (segment (start 69.15 53.34) (end 67.47 53.34) (width 1.5) (layer "F.Cu") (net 15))
 (segment (start 69.15 58.42) (end 67.47 58.42) (width 1.5) (layer "F.Cu") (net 13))
 (segment (start 70.42 59.69) (end 69.15 58.42) (width 1.5) (layer "F.Cu") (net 13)))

